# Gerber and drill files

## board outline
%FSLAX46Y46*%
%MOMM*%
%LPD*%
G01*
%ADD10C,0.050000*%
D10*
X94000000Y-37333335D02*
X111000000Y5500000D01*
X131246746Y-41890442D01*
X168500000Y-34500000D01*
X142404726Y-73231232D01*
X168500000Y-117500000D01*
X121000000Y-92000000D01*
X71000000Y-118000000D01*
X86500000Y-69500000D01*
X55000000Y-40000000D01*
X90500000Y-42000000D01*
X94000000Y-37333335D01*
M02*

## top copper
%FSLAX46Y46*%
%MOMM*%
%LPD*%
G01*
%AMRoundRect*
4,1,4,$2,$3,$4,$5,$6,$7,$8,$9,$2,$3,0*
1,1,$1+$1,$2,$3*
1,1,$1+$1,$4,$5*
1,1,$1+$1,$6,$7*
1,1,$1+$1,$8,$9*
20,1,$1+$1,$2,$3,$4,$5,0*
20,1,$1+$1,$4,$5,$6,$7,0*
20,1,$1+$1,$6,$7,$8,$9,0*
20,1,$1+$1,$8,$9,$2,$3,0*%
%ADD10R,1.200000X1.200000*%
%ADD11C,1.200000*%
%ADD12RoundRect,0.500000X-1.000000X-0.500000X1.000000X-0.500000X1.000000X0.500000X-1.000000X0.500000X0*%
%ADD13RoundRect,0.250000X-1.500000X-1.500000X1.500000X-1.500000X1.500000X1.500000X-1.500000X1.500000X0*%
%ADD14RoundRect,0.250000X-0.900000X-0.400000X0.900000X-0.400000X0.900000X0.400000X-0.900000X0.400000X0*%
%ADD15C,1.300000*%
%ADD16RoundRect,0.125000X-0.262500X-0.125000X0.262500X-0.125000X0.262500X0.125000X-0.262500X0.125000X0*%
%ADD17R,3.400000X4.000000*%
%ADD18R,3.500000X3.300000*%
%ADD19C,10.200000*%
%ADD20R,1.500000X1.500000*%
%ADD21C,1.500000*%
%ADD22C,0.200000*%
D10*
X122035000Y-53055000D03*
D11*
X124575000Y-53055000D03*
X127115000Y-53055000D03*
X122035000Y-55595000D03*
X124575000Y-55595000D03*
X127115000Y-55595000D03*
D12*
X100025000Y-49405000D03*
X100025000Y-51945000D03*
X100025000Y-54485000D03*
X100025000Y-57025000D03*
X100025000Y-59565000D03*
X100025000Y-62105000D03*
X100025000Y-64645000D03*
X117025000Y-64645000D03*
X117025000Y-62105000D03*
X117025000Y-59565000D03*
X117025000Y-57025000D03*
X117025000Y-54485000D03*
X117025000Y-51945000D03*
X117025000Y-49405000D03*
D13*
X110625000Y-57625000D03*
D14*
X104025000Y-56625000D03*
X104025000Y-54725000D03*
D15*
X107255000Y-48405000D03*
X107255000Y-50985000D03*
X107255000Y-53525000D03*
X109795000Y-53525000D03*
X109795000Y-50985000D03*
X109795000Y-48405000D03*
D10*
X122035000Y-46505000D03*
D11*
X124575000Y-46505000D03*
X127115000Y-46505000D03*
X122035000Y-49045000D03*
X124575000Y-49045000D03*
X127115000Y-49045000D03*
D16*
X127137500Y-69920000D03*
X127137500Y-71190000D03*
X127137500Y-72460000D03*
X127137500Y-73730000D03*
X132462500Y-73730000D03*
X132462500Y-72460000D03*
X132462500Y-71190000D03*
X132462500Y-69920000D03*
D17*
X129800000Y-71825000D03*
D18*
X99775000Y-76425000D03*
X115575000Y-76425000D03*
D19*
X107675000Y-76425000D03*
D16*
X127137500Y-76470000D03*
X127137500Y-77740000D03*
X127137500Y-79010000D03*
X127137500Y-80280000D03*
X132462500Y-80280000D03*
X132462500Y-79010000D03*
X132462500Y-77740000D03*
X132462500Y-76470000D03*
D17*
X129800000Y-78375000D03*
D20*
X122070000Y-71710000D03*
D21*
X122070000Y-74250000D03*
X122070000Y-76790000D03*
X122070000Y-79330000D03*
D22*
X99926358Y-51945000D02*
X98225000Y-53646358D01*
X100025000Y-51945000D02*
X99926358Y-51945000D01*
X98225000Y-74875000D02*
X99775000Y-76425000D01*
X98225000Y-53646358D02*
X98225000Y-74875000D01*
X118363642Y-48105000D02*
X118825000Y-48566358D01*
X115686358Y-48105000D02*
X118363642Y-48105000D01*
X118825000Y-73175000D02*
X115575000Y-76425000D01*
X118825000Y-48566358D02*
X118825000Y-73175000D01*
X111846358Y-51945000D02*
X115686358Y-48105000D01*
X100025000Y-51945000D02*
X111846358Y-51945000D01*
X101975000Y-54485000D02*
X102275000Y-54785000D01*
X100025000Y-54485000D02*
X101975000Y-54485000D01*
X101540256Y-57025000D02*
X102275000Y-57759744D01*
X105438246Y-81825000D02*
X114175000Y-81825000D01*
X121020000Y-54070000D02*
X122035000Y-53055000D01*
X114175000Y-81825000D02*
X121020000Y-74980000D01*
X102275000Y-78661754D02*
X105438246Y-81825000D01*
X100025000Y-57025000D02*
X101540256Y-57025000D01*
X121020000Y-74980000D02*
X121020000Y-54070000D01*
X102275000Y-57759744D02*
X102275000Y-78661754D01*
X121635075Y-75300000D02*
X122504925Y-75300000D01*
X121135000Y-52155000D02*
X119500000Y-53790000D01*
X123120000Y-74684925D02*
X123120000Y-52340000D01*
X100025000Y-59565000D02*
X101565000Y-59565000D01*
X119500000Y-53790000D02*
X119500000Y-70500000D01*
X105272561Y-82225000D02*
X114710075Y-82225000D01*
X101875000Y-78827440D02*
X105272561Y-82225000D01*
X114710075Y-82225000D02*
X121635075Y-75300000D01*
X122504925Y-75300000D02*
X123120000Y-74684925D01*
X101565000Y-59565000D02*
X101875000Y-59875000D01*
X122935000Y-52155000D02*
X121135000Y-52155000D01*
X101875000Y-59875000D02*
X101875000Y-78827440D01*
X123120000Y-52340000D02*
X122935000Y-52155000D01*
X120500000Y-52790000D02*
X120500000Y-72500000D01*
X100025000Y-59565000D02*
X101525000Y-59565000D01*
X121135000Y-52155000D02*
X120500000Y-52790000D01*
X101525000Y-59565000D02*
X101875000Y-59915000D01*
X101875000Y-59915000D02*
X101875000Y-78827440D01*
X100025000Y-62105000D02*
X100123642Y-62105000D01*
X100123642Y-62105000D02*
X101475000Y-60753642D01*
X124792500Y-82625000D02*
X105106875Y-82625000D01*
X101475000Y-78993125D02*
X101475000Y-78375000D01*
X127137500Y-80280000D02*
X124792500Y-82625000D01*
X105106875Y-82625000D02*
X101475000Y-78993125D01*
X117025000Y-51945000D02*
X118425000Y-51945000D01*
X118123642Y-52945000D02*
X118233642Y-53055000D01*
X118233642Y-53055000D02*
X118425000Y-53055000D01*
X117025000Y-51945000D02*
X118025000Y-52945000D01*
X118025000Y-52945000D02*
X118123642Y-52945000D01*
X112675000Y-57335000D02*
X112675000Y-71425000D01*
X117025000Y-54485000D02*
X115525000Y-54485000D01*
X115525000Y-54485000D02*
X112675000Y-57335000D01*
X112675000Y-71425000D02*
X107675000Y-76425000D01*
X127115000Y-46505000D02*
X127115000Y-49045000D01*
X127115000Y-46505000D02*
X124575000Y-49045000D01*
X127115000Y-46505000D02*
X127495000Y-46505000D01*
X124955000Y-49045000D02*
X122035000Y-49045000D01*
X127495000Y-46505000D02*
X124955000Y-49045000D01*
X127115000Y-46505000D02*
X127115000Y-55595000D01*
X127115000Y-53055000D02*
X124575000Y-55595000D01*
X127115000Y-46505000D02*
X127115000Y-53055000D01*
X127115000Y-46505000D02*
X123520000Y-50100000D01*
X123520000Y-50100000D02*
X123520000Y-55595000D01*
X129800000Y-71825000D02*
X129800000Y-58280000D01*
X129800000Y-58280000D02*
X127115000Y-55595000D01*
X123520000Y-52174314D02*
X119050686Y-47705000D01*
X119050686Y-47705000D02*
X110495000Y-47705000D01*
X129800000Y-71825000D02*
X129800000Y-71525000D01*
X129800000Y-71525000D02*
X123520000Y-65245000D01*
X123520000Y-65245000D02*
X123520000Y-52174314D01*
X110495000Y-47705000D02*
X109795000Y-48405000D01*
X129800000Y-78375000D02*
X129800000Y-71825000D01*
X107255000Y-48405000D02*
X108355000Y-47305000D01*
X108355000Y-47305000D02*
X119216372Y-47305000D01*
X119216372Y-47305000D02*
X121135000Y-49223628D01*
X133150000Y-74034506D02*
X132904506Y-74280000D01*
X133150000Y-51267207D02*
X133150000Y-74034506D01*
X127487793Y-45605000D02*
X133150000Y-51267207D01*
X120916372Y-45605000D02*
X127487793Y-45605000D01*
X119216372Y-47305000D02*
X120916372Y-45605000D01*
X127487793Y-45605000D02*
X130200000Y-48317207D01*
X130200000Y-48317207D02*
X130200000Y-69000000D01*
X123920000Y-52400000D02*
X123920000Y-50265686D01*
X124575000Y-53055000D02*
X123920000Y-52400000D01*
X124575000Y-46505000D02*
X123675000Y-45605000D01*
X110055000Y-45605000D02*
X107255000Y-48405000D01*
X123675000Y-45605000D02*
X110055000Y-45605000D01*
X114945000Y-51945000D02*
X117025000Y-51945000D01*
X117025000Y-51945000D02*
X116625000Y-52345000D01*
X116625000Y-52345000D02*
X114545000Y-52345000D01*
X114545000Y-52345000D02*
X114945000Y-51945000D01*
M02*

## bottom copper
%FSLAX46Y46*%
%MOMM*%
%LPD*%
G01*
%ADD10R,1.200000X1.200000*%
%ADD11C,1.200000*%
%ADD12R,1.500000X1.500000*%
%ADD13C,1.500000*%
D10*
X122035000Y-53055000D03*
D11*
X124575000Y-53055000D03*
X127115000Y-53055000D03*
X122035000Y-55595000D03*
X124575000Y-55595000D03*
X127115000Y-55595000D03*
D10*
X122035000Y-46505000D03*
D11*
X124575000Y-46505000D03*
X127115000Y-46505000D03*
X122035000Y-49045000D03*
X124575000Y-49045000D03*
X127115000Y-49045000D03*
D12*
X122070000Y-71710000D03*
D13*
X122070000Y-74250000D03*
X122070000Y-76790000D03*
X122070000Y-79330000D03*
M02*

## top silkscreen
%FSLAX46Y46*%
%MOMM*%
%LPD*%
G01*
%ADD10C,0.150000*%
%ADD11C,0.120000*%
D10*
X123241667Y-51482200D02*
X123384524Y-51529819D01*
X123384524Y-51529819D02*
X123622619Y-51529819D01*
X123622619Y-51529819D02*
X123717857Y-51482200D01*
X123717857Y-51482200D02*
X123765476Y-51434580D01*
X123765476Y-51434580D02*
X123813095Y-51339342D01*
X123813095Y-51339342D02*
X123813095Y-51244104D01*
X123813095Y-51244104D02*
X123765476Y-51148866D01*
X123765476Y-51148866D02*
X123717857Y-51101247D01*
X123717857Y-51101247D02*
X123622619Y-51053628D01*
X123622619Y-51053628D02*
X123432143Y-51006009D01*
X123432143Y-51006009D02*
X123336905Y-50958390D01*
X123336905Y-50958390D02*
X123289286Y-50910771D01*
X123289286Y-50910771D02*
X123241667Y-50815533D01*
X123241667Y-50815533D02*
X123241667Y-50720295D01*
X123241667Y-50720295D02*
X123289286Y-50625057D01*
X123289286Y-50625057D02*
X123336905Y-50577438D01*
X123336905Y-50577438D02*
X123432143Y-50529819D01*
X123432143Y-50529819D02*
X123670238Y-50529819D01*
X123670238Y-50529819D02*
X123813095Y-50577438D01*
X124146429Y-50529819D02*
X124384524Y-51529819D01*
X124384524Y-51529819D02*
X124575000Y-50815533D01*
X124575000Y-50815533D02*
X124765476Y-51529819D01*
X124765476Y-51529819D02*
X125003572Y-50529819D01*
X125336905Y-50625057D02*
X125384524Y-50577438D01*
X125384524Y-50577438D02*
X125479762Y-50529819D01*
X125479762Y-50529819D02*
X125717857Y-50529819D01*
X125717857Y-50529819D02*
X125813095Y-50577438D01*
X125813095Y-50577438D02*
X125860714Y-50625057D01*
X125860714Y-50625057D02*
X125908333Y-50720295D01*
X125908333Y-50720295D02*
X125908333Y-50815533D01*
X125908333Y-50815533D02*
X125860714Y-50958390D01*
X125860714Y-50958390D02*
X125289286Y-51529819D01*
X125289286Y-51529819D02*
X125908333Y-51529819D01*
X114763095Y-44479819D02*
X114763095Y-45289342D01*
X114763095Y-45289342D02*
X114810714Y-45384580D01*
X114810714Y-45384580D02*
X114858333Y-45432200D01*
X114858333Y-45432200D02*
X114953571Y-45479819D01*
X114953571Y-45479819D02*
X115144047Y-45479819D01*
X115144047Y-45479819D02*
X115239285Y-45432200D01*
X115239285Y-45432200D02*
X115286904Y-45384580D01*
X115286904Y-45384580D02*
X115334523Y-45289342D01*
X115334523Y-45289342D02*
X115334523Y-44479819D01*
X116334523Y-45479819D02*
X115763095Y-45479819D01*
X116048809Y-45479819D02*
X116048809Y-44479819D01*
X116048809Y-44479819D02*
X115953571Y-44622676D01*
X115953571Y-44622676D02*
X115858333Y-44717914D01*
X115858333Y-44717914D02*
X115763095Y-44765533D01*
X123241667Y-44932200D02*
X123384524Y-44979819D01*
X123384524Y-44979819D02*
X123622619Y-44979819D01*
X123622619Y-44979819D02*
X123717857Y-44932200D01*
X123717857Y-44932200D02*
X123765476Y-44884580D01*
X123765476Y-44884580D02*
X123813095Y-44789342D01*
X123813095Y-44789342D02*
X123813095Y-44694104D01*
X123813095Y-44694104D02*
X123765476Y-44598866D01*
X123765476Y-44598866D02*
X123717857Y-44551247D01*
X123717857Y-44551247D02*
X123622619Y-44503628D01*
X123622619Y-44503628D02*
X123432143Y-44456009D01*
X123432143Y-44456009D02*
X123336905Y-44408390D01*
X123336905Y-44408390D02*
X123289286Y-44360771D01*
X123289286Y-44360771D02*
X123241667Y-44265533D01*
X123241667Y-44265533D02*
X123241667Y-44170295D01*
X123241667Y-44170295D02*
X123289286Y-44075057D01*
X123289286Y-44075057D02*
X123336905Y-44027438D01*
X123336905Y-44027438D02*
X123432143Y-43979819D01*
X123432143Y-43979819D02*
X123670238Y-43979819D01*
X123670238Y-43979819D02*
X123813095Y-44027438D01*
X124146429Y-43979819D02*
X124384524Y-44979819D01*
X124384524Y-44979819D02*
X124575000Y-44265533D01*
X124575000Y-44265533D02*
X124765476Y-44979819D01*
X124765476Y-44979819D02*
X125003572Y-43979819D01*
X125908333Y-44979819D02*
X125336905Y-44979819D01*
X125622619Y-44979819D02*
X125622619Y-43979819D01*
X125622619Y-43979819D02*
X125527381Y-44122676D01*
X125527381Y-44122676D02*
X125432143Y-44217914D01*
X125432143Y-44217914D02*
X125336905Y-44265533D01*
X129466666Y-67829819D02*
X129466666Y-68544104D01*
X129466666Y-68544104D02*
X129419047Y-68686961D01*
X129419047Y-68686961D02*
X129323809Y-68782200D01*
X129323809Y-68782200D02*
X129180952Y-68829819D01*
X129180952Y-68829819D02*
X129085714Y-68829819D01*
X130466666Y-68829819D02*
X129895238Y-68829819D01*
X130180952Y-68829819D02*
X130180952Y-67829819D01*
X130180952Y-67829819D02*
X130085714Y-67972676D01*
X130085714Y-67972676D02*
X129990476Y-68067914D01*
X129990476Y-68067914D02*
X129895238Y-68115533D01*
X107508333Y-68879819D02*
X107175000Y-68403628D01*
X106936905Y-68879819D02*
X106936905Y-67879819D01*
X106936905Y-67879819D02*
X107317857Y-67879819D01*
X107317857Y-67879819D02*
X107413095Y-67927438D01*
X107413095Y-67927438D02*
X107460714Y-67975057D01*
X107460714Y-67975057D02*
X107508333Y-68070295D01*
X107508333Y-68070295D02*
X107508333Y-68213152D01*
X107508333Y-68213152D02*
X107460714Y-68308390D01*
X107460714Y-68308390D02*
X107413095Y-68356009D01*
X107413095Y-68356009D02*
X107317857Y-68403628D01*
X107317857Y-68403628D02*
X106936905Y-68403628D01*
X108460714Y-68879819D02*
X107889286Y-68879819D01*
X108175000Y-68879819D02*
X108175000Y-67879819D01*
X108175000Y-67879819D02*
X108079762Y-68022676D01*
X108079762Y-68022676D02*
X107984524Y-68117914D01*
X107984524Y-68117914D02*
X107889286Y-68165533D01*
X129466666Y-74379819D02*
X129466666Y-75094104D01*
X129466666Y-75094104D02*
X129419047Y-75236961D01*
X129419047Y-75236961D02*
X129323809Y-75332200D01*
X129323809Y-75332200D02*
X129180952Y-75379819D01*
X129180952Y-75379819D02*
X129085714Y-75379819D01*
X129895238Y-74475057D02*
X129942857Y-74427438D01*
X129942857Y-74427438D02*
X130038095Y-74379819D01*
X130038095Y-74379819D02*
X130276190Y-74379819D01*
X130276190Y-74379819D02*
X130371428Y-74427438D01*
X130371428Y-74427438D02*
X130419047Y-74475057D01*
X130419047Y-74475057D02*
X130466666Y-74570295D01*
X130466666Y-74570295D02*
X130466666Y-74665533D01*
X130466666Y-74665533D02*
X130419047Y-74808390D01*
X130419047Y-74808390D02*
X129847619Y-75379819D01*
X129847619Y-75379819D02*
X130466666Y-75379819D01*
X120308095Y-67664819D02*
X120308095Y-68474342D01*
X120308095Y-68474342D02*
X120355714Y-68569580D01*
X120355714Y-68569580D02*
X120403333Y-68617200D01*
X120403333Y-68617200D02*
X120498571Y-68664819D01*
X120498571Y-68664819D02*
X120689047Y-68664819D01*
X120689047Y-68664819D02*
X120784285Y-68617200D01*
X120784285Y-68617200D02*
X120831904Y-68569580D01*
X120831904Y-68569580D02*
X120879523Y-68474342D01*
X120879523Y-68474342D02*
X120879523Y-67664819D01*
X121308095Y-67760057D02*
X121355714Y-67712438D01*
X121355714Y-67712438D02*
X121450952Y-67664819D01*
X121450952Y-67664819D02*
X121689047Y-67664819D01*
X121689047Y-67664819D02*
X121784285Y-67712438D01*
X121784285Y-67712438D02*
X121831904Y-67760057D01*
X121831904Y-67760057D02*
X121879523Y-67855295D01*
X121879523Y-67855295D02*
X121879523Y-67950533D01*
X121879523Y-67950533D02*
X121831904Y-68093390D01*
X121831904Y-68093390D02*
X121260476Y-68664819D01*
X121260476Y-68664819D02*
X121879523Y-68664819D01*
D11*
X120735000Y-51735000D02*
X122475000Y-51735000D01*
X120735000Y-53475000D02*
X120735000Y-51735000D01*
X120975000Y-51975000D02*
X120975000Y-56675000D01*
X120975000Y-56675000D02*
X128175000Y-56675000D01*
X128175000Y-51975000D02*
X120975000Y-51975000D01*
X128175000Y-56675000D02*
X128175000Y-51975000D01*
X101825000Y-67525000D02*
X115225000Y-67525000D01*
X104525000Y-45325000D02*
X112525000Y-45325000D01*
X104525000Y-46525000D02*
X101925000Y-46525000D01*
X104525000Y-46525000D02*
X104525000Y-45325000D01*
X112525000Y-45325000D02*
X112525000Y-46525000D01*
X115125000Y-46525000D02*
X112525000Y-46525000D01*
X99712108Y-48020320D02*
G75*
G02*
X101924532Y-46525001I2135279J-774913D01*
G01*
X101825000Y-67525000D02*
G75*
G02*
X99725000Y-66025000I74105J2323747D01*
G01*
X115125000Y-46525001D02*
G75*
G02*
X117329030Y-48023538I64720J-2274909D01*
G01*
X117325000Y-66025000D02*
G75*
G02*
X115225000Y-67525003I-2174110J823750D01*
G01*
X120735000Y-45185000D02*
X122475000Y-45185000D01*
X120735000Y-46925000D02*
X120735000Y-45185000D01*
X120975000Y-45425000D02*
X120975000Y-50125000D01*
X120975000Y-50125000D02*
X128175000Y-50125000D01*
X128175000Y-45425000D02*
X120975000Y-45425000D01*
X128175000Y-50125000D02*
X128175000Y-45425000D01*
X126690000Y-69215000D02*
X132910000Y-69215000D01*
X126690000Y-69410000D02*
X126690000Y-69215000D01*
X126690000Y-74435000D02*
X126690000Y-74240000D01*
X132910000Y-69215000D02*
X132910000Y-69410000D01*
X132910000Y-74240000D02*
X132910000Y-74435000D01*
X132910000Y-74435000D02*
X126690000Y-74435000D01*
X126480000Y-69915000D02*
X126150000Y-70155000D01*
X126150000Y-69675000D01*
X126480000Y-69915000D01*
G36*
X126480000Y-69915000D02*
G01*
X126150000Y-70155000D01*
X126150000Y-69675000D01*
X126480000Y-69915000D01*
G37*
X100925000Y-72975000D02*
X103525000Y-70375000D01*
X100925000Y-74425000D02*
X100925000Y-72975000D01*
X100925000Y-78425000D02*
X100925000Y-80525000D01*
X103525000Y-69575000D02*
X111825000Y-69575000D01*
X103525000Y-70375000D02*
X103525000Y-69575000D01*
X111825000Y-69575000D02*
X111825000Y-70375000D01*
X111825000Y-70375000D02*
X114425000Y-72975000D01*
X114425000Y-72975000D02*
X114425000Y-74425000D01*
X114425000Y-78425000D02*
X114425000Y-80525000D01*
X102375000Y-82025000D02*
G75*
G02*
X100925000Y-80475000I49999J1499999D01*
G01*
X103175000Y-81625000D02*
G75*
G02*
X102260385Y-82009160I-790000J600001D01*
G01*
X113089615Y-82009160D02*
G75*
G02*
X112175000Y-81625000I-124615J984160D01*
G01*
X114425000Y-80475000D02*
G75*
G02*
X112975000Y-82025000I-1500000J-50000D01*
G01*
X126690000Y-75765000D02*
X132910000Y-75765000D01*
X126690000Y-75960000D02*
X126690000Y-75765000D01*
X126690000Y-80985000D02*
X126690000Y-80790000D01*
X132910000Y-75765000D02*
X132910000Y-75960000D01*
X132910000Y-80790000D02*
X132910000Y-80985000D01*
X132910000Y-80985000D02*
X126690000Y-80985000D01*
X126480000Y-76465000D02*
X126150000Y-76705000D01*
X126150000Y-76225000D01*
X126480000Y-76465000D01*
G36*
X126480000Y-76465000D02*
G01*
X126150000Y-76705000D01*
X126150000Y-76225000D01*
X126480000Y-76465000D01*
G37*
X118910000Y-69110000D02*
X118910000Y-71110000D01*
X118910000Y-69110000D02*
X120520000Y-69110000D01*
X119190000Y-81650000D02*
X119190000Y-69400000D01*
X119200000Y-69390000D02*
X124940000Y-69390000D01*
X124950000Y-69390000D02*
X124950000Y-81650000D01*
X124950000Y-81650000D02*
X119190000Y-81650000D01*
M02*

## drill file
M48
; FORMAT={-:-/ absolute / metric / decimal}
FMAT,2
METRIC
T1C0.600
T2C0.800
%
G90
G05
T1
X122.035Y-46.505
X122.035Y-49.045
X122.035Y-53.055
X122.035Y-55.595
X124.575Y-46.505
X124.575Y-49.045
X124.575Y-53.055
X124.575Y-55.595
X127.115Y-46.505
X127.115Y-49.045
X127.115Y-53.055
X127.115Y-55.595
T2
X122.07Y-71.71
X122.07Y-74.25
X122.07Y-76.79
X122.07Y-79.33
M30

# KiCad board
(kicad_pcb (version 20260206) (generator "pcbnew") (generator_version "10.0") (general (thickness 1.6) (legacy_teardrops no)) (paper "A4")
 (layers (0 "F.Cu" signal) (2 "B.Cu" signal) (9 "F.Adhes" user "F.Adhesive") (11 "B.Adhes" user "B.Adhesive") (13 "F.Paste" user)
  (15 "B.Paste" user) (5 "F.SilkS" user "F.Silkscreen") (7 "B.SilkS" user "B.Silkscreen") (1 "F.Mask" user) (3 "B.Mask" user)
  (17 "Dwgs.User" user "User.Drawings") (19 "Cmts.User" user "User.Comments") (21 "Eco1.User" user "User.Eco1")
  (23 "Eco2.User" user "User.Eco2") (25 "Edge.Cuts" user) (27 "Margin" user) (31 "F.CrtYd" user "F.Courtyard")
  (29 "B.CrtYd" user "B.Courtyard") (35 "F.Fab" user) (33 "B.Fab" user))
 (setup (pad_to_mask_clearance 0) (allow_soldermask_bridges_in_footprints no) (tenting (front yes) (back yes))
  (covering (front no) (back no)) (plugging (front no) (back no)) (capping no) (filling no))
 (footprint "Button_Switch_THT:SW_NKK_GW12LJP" (layer "F.Cu") (at 122.035 53.055)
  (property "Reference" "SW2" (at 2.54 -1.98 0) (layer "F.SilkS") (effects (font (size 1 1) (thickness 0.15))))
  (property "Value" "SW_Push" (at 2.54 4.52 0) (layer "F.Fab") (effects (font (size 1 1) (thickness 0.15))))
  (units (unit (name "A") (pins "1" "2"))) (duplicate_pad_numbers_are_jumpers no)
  (fp_line (start -1.3 -1.32) (end 0.44 -1.32) (stroke (width 0.12) (type solid)) (layer "F.SilkS"))
  (fp_line (start -1.3 0.42) (end -1.3 -1.32) (stroke (width 0.12) (type solid)) (layer "F.SilkS"))
  (fp_line (start -1.06 -1.08) (end -1.06 3.62) (stroke (width 0.12) (type solid)) (layer "F.SilkS"))
  (fp_line (start -1.06 3.62) (end 6.14 3.62) (stroke (width 0.12) (type solid)) (layer "F.SilkS"))
  (fp_line (start 6.14 -1.08) (end -1.06 -1.08) (stroke (width 0.12) (type solid)) (layer "F.SilkS"))
  (fp_line (start 6.14 3.62) (end 6.14 -1.08) (stroke (width 0.12) (type solid)) (layer "F.SilkS"))
  (pad "1" thru_hole rect (at 0 0) (size 1.2 1.2) (drill 0.6) (layers "*.Cu" "*.Mask") (remove_unused_layers no) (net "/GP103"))
  (pad "2" thru_hole circle (at 2.54 0) (size 1.2 1.2) (drill 0.6) (layers "*.Cu" "*.Mask") (remove_unused_layers no) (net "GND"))
  (pad "3" thru_hole circle (at 5.08 0) (size 1.2 1.2) (drill 0.6) (layers "*.Cu" "*.Mask") (remove_unused_layers no))
  (pad "4" thru_hole circle (at 0 2.54) (size 1.2 1.2) (drill 0.6) (layers "*.Cu" "*.Mask") (remove_unused_layers no))
  (pad "5" thru_hole circle (at 2.54 2.54) (size 1.2 1.2) (drill 0.6) (layers "*.Cu" "*.Mask") (remove_unused_layers no))
  (pad "6" thru_hole circle (at 5.08 2.54) (size 1.2 1.2) (drill 0.6) (layers "*.Cu" "*.Mask") (remove_unused_layers no)))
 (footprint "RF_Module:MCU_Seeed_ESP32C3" (layer "F.Cu") (at 108.525 57.025)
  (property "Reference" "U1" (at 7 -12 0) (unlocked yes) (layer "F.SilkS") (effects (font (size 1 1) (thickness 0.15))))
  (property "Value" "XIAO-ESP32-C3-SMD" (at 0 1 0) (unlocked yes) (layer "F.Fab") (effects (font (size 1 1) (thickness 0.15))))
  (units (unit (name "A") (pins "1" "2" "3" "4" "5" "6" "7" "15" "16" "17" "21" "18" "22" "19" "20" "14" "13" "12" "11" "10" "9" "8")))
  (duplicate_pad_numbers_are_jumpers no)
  (fp_line (start -6.7 10.5) (end 6.7 10.5) (stroke (width 0.12) (type default)) (layer "F.SilkS"))
  (fp_line (start -4 -11.7) (end 4 -11.7) (stroke (width 0.12) (type default)) (layer "F.SilkS"))
  (fp_line (start -4 -10.5) (end -6.6 -10.5) (stroke (width 0.12) (type default)) (layer "F.SilkS"))
  (fp_line (start -4 -10.5) (end -4 -11.7) (stroke (width 0.12) (type default)) (layer "F.SilkS"))
  (fp_line (start 4 -11.7) (end 4 -10.5) (stroke (width 0.12) (type default)) (layer "F.SilkS"))
  (fp_line (start 6.6 -10.5) (end 4 -10.5) (stroke (width 0.12) (type default)) (layer "F.SilkS"))
  (fp_arc (start -8.812892 -9.00468) (mid -7.949609 -10.111769) (end -6.600468 -10.499999) (stroke (width 0.12) (type default))
   (layer "F.SilkS"))
  (fp_arc (start -6.7 10.5) (mid -7.977232 10.068125) (end -8.8 9) (stroke (width 0.12) (type default)) (layer "F.SilkS"))
  (fp_arc (start 6.6 -10.499999) (mid 7.944325 -10.107116) (end 8.804034 -9.001464) (stroke (width 0.12) (type default)) (layer "F.SilkS"))
  (fp_arc (start 8.8 9) (mid 7.977232 10.068125) (end 6.7 10.5) (stroke (width 0.12) (type default)) (layer "F.SilkS"))
  (pad "" smd roundrect (at 1.1 -0.4) (size 1.5 1.5) (layers "F.Paste") (roundrect_rratio 0.1666666667))
  (pad "" smd roundrect (at 1.1 1.6) (size 1.5 1.5) (layers "F.Paste") (roundrect_rratio 0.1666666667))
  (pad "" smd roundrect (at 3.1 -0.4) (size 1.5 1.5) (layers "F.Paste") (roundrect_rratio 0.1666666667))
  (pad "" smd roundrect (at 3.1 1.6) (size 1.5 1.5) (layers "F.Paste") (roundrect_rratio 0.1666666667))
  (pad "1" smd roundrect (at -8.5 -7.62) (size 3 2) (layers "F.Cu" "F.Mask" "F.Paste") (roundrect_rratio 0.25)
   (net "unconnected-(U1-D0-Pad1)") (thermal_bridge_angle 45))
  (pad "2" smd roundrect (at -8.5 -5.08) (size 3 2) (layers "F.Cu" "F.Mask" "F.Paste") (roundrect_rratio 0.25) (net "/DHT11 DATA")
   (thermal_bridge_angle 45))
  (pad "3" smd roundrect (at -8.5 -2.54) (size 3 2) (layers "F.Cu" "F.Mask" "F.Paste") (roundrect_rratio 0.25) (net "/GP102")
   (thermal_bridge_angle 45))
  (pad "4" smd roundrect (at -8.5 0) (size 3 2) (layers "F.Cu" "F.Mask" "F.Paste") (roundrect_rratio 0.25) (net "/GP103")
   (thermal_bridge_angle 45))
  (pad "5" smd roundrect (at -8.5 2.54) (size 3 2) (layers "F.Cu" "F.Mask" "F.Paste") (roundrect_rratio 0.25) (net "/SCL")
   (thermal_bridge_angle 45))
  (pad "6" smd roundrect (at -8.5 5.08) (size 3 2) (layers "F.Cu" "F.Mask" "F.Paste") (roundrect_rratio 0.25) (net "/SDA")
   (thermal_bridge_angle 45))
  (pad "7" smd roundrect (at -8.5 7.62) (size 3 2) (layers "F.Cu" "F.Mask" "F.Paste") (roundrect_rratio 0.25)
   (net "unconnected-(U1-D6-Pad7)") (thermal_bridge_angle 45))
  (pad "8" smd roundrect (at 8.5 7.62) (size 3 2) (layers "F.Cu" "F.Mask" "F.Paste") (roundrect_rratio 0.25)
   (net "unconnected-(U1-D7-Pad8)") (thermal_bridge_angle 45))
  (pad "9" smd roundrect (at 8.5 5.08) (size 3 2) (layers "F.Cu" "F.Mask" "F.Paste") (roundrect_rratio 0.25)
   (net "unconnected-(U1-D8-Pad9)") (thermal_bridge_angle 45))
  (pad "10" smd roundrect (at 8.5 2.54) (size 3 2) (layers "F.Cu" "F.Mask" "F.Paste") (roundrect_rratio 0.25)
   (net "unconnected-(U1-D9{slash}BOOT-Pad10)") (thermal_bridge_angle 45))
  (pad "11" smd roundrect (at 8.5 0) (size 3 2) (layers "F.Cu" "F.Mask" "F.Paste") (roundrect_rratio 0.25)
   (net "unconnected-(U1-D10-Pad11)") (thermal_bridge_angle 45))
  (pad "12" smd roundrect (at 8.5 -2.54) (size 3 2) (layers "F.Cu" "F.Mask" "F.Paste") (roundrect_rratio 0.25) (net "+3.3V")
   (thermal_bridge_angle 45))
  (pad "13" smd roundrect (at 8.5 -5.08) (size 3 2) (layers "F.Cu" "F.Mask" "F.Paste") (roundrect_rratio 0.25) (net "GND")
   (thermal_bridge_angle 45))
  (pad "14" smd roundrect (at 8.5 -7.62) (size 3 2) (layers "F.Cu" "F.Mask" "F.Paste") (roundrect_rratio 0.25) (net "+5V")
   (thermal_bridge_angle 45))
  (pad "15" smd roundrect (at 2.1 0.6) (size 3.5 3.5) (layers "F.Cu" "F.Mask") (roundrect_rratio 0.07142857143)
   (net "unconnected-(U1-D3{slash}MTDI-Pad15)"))
  (pad "16" smd roundrect (at -4.5 -0.4) (size 2.3 1.3) (layers "F.Cu" "F.Mask" "F.Paste") (roundrect_rratio 0.1923076923)
   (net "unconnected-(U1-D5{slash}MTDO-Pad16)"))
  (pad "17" smd roundrect (at -4.5 -2.3) (size 2.3 1.3) (layers "F.Cu" "F.Mask" "F.Paste") (roundrect_rratio 0.1923076923)
   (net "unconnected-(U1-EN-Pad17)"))
  (pad "18" smd circle (at -1.27 -8.62) (size 1.3 1.3) (layers "F.Cu" "F.Mask" "F.Paste") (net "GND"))
  (pad "19" smd circle (at -1.27 -6.04) (size 1.3 1.3) (layers "F.Cu" "F.Mask" "F.Paste") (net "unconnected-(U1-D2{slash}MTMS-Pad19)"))
  (pad "20" smd circle (at -1.27 -3.5) (size 1.3 1.3) (layers "F.Cu" "F.Mask" "F.Paste") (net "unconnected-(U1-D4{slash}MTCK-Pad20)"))
  (pad "21" smd circle (at 1.27 -3.5) (size 1.3 1.3) (layers "F.Cu" "F.Mask" "F.Paste") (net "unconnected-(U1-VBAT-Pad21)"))
  (pad "22" smd circle (at 1.27 -6.04) (size 1.3 1.3) (layers "F.Cu" "F.Mask" "F.Paste") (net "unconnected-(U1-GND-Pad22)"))
  (pad "23" smd circle (at 1.27 -8.62) (size 1.3 1.3) (layers "F.Cu" "F.Mask" "F.Paste")))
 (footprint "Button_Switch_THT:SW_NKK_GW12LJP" (layer "F.Cu") (at 122.035 46.505)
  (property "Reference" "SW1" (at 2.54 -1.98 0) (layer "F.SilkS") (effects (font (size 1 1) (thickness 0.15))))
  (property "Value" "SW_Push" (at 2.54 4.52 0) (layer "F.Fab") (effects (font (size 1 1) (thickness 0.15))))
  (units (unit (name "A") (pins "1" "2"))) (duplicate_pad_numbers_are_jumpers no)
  (fp_line (start -1.3 -1.32) (end 0.44 -1.32) (stroke (width 0.12) (type solid)) (layer "F.SilkS"))
  (fp_line (start -1.3 0.42) (end -1.3 -1.32) (stroke (width 0.12) (type solid)) (layer "F.SilkS"))
  (fp_line (start -1.06 -1.08) (end -1.06 3.62) (stroke (width 0.12) (type solid)) (layer "F.SilkS"))
  (fp_line (start -1.06 3.62) (end 6.14 3.62) (stroke (width 0.12) (type solid)) (layer "F.SilkS"))
  (fp_line (start 6.14 -1.08) (end -1.06 -1.08) (stroke (width 0.12) (type solid)) (layer "F.SilkS"))
  (fp_line (start 6.14 3.62) (end 6.14 -1.08) (stroke (width 0.12) (type solid)) (layer "F.SilkS"))
  (pad "1" thru_hole rect (at 0 0) (size 1.2 1.2) (drill 0.6) (layers "*.Cu" "*.Mask") (remove_unused_layers no) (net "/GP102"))
  (pad "2" thru_hole circle (at 2.54 0) (size 1.2 1.2) (drill 0.6) (layers "*.Cu" "*.Mask") (remove_unused_layers no) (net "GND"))
  (pad "3" thru_hole circle (at 5.08 0) (size 1.2 1.2) (drill 0.6) (layers "*.Cu" "*.Mask") (remove_unused_layers no))
  (pad "4" thru_hole circle (at 0 2.54) (size 1.2 1.2) (drill 0.6) (layers "*.Cu" "*.Mask") (remove_unused_layers no))
  (pad "5" thru_hole circle (at 2.54 2.54) (size 1.2 1.2) (drill 0.6) (layers "*.Cu" "*.Mask") (remove_unused_layers no))
  (pad "6" thru_hole circle (at 5.08 2.54) (size 1.2 1.2) (drill 0.6) (layers "*.Cu" "*.Mask") (remove_unused_layers no)))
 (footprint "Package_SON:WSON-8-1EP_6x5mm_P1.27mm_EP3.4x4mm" (layer "F.Cu") (at 129.8 71.825)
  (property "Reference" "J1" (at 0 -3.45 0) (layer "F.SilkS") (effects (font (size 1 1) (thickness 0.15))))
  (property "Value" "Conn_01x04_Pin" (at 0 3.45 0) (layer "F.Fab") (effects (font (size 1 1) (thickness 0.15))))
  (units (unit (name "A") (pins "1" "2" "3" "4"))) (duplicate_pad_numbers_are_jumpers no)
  (fp_line (start -3.11 -2.61) (end 3.11 -2.61) (stroke (width 0.12) (type solid)) (layer "F.SilkS"))
  (fp_line (start -3.11 -2.415) (end -3.11 -2.61) (stroke (width 0.12) (type solid)) (layer "F.SilkS"))
  (fp_line (start -3.11 2.61) (end -3.11 2.415) (stroke (width 0.12) (type solid)) (layer "F.SilkS"))
  (fp_line (start 3.11 -2.61) (end 3.11 -2.415) (stroke (width 0.12) (type solid)) (layer "F.SilkS"))
  (fp_line (start 3.11 2.415) (end 3.11 2.61) (stroke (width 0.12) (type solid)) (layer "F.SilkS"))
  (fp_line (start 3.11 2.61) (end -3.11 2.61) (stroke (width 0.12) (type solid)) (layer "F.SilkS"))
  (fp_poly (pts (xy -3.32 -1.91) (xy -3.65 -1.67) (xy -3.65 -2.15)) (stroke (width 0.12) (type solid)) (fill yes) (layer "F.SilkS"))
  (pad "" smd roundrect (at -0.85 -1) (size 1.37 1.61) (layers "F.Paste") (roundrect_rratio 0.182482))
  (pad "" smd roundrect (at -0.85 1) (size 1.37 1.61) (layers "F.Paste") (roundrect_rratio 0.182482))
  (pad "" smd roundrect (at 0.85 -1) (size 1.37 1.61) (layers "F.Paste") (roundrect_rratio 0.182482))
  (pad "" smd roundrect (at 0.85 1) (size 1.37 1.61) (layers "F.Paste") (roundrect_rratio 0.182482))
  (pad "1" smd roundrect (at -2.6625 -1.905) (size 0.775 0.5) (layers "F.Cu" "F.Mask" "F.Paste") (roundrect_rratio 0.25) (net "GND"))
  (pad "2" smd roundrect (at -2.6625 -0.635) (size 0.775 0.5) (layers "F.Cu" "F.Mask" "F.Paste") (roundrect_rratio 0.25) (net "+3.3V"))
  (pad "3" smd roundrect (at -2.6625 0.635) (size 0.775 0.5) (layers "F.Cu" "F.Mask" "F.Paste") (roundrect_rratio 0.25) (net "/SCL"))
  (pad "4" smd roundrect (at -2.6625 1.905) (size 0.775 0.5) (layers "F.Cu" "F.Mask" "F.Paste") (roundrect_rratio 0.25) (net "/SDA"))
  (pad "5" smd roundrect (at 2.6625 1.905) (size 0.775 0.5) (layers "F.Cu" "F.Mask" "F.Paste") (roundrect_rratio 0.25))
  (pad "6" smd roundrect (at 2.6625 0.635) (size 0.775 0.5) (layers "F.Cu" "F.Mask" "F.Paste") (roundrect_rratio 0.25))
  (pad "7" smd roundrect (at 2.6625 -0.635) (size 0.775 0.5) (layers "F.Cu" "F.Mask" "F.Paste") (roundrect_rratio 0.25))
  (pad "8" smd roundrect (at 2.6625 -1.905) (size 0.775 0.5) (layers "F.Cu" "F.Mask" "F.Paste") (roundrect_rratio 0.25))
  (pad "9" smd rect (at 0 0) (size 3.4 4) (layers "F.Cu" "F.Mask") (zone_connect 2)))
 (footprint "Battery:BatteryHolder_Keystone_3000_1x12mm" (layer "F.Cu") (at 107.675 76.425)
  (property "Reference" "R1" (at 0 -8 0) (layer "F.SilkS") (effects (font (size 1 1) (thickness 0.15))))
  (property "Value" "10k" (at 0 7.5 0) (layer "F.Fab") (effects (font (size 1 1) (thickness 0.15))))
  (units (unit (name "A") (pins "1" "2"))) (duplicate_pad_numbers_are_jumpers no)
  (fp_line (start -6.75 -3.45) (end -4.15 -6.05) (stroke (width 0.12) (type solid)) (layer "F.SilkS"))
  (fp_line (start -6.75 -2) (end -6.75 -3.45) (stroke (width 0.12) (type solid)) (layer "F.SilkS"))
  (fp_line (start -6.75 2) (end -6.75 4.1) (stroke (width 0.12) (type solid)) (layer "F.SilkS"))
  (fp_line (start -4.15 -6.85) (end 4.15 -6.85) (stroke (width 0.12) (type solid)) (layer "F.SilkS"))
  (fp_line (start -4.15 -6.05) (end -4.15 -6.85) (stroke (width 0.12) (type solid)) (layer "F.SilkS"))
  (fp_line (start 4.15 -6.85) (end 4.15 -6.05) (stroke (width 0.12) (type solid)) (layer "F.SilkS"))
  (fp_line (start 4.15 -6.05) (end 6.75 -3.45) (stroke (width 0.12) (type solid)) (layer "F.SilkS"))
  (fp_line (start 6.75 -3.45) (end 6.75 -2) (stroke (width 0.12) (type solid)) (layer "F.SilkS"))
  (fp_line (start 6.75 2) (end 6.75 4.1) (stroke (width 0.12) (type solid)) (layer "F.SilkS"))
  (fp_arc (start -5.3 5.6) (mid -6.346016 5.125305) (end -6.75 4.05) (stroke (width 0.12) (type solid)) (layer "F.SilkS"))
  (fp_arc (start -4.5 5.2) (mid -4.90584 5.514615) (end -5.414615 5.58416) (stroke (width 0.12) (type solid)) (layer "F.SilkS"))
  (fp_arc (start 5.414615 5.58416) (mid 4.90584 5.514615) (end 4.5 5.2) (stroke (width 0.12) (type solid)) (layer "F.SilkS"))
  (fp_arc (start 6.75 4.05) (mid 6.346016 5.125305) (end 5.3 5.6) (stroke (width 0.12) (type solid)) (layer "F.SilkS"))
  (pad "1" smd rect (at -7.9 0) (size 3.5 3.3) (layers "F.Cu" "F.Mask" "F.Paste") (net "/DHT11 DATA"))
  (pad "1" smd rect (at 7.9 0) (size 3.5 3.3) (layers "F.Cu" "F.Mask" "F.Paste") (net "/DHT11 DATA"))
  (pad "2" smd circle (at 0 0) (size 10.2 10.2) (layers "F.Cu" "F.Mask") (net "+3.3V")))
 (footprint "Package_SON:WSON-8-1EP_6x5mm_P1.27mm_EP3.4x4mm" (layer "F.Cu") (at 129.8 78.375)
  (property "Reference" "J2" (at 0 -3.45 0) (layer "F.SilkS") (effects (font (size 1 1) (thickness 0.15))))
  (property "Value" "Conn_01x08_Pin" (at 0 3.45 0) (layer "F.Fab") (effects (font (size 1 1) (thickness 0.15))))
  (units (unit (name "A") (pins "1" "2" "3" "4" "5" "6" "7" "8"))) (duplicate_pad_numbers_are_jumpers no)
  (fp_line (start -3.11 -2.61) (end 3.11 -2.61) (stroke (width 0.12) (type solid)) (layer "F.SilkS"))
  (fp_line (start -3.11 -2.415) (end -3.11 -2.61) (stroke (width 0.12) (type solid)) (layer "F.SilkS"))
  (fp_line (start -3.11 2.61) (end -3.11 2.415) (stroke (width 0.12) (type solid)) (layer "F.SilkS"))
  (fp_line (start 3.11 -2.61) (end 3.11 -2.415) (stroke (width 0.12) (type solid)) (layer "F.SilkS"))
  (fp_line (start 3.11 2.415) (end 3.11 2.61) (stroke (width 0.12) (type solid)) (layer "F.SilkS"))
  (fp_line (start 3.11 2.61) (end -3.11 2.61) (stroke (width 0.12) (type solid)) (layer "F.SilkS"))
  (fp_poly (pts (xy -3.32 -1.91) (xy -3.65 -1.67) (xy -3.65 -2.15)) (stroke (width 0.12) (type solid)) (fill yes) (layer "F.SilkS"))
  (pad "" smd roundrect (at -0.85 -1) (size 1.37 1.61) (layers "F.Paste") (roundrect_rratio 0.182482))
  (pad "" smd roundrect (at -0.85 1) (size 1.37 1.61) (layers "F.Paste") (roundrect_rratio 0.182482))
  (pad "" smd roundrect (at 0.85 -1) (size 1.37 1.61) (layers "F.Paste") (roundrect_rratio 0.182482))
  (pad "" smd roundrect (at 0.85 1) (size 1.37 1.61) (layers "F.Paste") (roundrect_rratio 0.182482))
  (pad "1" smd roundrect (at -2.6625 -1.905) (size 0.775 0.5) (layers "F.Cu" "F.Mask" "F.Paste") (roundrect_rratio 0.25) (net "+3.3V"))
  (pad "2" smd roundrect (at -2.6625 -0.635) (size 0.775 0.5) (layers "F.Cu" "F.Mask" "F.Paste") (roundrect_rratio 0.25) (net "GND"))
  (pad "3" smd roundrect (at -2.6625 0.635) (size 0.775 0.5) (layers "F.Cu" "F.Mask" "F.Paste") (roundrect_rratio 0.25) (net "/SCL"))
  (pad "4" smd roundrect (at -2.6625 1.905) (size 0.775 0.5) (layers "F.Cu" "F.Mask" "F.Paste") (roundrect_rratio 0.25) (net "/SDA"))
  (pad "5" smd roundrect (at 2.6625 1.905) (size 0.775 0.5) (layers "F.Cu" "F.Mask" "F.Paste") (roundrect_rratio 0.25)
   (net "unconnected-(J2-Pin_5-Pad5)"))
  (pad "6" smd roundrect (at 2.6625 0.635) (size 0.775 0.5) (layers "F.Cu" "F.Mask" "F.Paste") (roundrect_rratio 0.25)
   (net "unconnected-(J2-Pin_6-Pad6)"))
  (pad "7" smd roundrect (at 2.6625 -0.635) (size 0.775 0.5) (layers "F.Cu" "F.Mask" "F.Paste") (roundrect_rratio 0.25)
   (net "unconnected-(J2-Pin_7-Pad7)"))
  (pad "8" smd roundrect (at 2.6625 -1.905) (size 0.775 0.5) (layers "F.Cu" "F.Mask" "F.Paste") (roundrect_rratio 0.25)
   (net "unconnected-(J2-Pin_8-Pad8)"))
  (pad "9" smd rect (at 0 0) (size 3.4 4) (layers "F.Cu" "F.Mask") (zone_connect 2)))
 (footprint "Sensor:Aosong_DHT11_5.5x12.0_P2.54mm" (layer "F.Cu") (at 122.07 71.71)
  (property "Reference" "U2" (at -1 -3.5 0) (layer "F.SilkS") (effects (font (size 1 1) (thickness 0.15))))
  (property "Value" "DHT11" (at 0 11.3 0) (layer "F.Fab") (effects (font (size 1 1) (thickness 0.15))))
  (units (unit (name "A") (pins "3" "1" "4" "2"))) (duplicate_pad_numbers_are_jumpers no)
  (fp_line (start -3.16 -2.6) (end -3.16 -0.6) (stroke (width 0.12) (type solid)) (layer "F.SilkS"))
  (fp_line (start -3.16 -2.6) (end -1.55 -2.6) (stroke (width 0.12) (type solid)) (layer "F.SilkS"))
  (fp_line (start -2.88 9.94) (end -2.88 -2.31) (stroke (width 0.12) (type solid)) (layer "F.SilkS"))
  (fp_line (start -2.87 -2.32) (end 2.87 -2.32) (stroke (width 0.12) (type solid)) (layer "F.SilkS"))
  (fp_line (start 2.88 -2.32) (end 2.88 9.94) (stroke (width 0.12) (type solid)) (layer "F.SilkS"))
  (fp_line (start 2.88 9.94) (end -2.88 9.94) (stroke (width 0.12) (type solid)) (layer "F.SilkS"))
  (pad "1" thru_hole rect (at 0 0) (size 1.5 1.5) (drill 0.8) (layers "*.Cu" "*.Mask") (remove_unused_layers no) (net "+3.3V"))
  (pad "2" thru_hole circle (at 0 2.54) (size 1.5 1.5) (drill 0.8) (layers "*.Cu" "*.Mask") (remove_unused_layers no) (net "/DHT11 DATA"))
  (pad "3" thru_hole circle (at 0 5.08) (size 1.5 1.5) (drill 0.8) (layers "*.Cu" "*.Mask") (remove_unused_layers no)
   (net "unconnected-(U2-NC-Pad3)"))
  (pad "4" thru_hole circle (at 0 7.62) (size 1.5 1.5) (drill 0.8) (layers "*.Cu" "*.Mask") (remove_unused_layers no) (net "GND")))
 (gr_poly
  (pts (xy 94 37.333335) (xy 111 -5.5) (xy 131.246746 41.890442) (xy 168.5 34.5) (xy 142.404726 73.231232) (xy 168.5 117.5) (xy 121 92)
   (xy 71 118) (xy 86.5 69.5) (xy 55 40) (xy 90.5 42))
  (stroke (width 0.05) (type solid)) (fill no) (layer "Edge.Cuts"))
 (segment (start 99.926358 51.945) (end 98.225 53.646358) (width 0.2) (layer "F.Cu") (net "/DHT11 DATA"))
 (segment (start 100.025 51.945) (end 99.926358 51.945) (width 0.2) (layer "F.Cu") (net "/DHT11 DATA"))
 (segment (start 98.225 74.875) (end 99.775 76.425) (width 0.2) (layer "F.Cu") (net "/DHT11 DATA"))
 (segment (start 98.225 53.646358) (end 98.225 74.875) (width 0.2) (layer "F.Cu") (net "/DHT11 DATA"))
 (segment (start 118.363642 48.105) (end 118.825 48.566358) (width 0.2) (layer "F.Cu") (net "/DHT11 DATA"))
 (segment (start 115.686358 48.105) (end 118.363642 48.105) (width 0.2) (layer "F.Cu") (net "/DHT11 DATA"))
 (segment (start 118.825 73.175) (end 115.575 76.425) (width 0.2) (layer "F.Cu") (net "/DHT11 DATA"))
 (segment (start 118.825 48.566358) (end 118.825 73.175) (width 0.2) (layer "F.Cu") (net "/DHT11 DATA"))
 (segment (start 111.846358 51.945) (end 115.686358 48.105) (width 0.2) (layer "F.Cu") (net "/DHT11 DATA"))
 (segment (start 100.025 51.945) (end 111.846358 51.945) (width 0.2) (layer "F.Cu") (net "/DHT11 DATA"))
 (segment (start 101.975 54.485) (end 102.275 54.785) (width 0.2) (layer "F.Cu") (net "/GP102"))
 (segment (start 100.025 54.485) (end 101.975 54.485) (width 0.2) (layer "F.Cu") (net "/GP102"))
 (segment (start 101.540256 57.025) (end 102.275 57.759744) (width 0.2) (layer "F.Cu") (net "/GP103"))
 (segment (start 105.438246 81.825) (end 114.175 81.825) (width 0.2) (layer "F.Cu") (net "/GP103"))
 (segment (start 121.02 54.07) (end 122.035 53.055) (width 0.2) (layer "F.Cu") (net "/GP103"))
 (segment (start 114.175 81.825) (end 121.02 74.98) (width 0.2) (layer "F.Cu") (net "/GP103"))
 (segment (start 102.275 78.661754) (end 105.438246 81.825) (width 0.2) (layer "F.Cu") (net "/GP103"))
 (segment (start 100.025 57.025) (end 101.540256 57.025) (width 0.2) (layer "F.Cu") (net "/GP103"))
 (segment (start 121.02 74.98) (end 121.02 54.07) (width 0.2) (layer "F.Cu") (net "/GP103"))
 (segment (start 102.275 57.759744) (end 102.275 78.661754) (width 0.2) (layer "F.Cu") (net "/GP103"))
 (segment (start 121.635075 75.3) (end 122.504925 75.3) (width 0.2) (layer "F.Cu") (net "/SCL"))
 (segment (start 121.135 52.155) (end 119.5 53.79) (width 0.2) (layer "F.Cu") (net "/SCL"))
 (segment (start 123.12 74.684925) (end 123.12 52.34) (width 0.2) (layer "F.Cu") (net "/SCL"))
 (segment (start 100.025 59.565) (end 101.565 59.565) (width 0.2) (layer "F.Cu") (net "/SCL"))
 (segment (start 119.5 53.79) (end 119.5 70.5) (width 0.2) (layer "F.Cu") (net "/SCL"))
 (segment (start 105.272561 82.225) (end 114.710075 82.225) (width 0.2) (layer "F.Cu") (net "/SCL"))
 (segment (start 101.875 78.82744) (end 105.272561 82.225) (width 0.2) (layer "F.Cu") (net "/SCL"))
 (segment (start 114.710075 82.225) (end 121.635075 75.3) (width 0.2) (layer "F.Cu") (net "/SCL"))
 (segment (start 122.504925 75.3) (end 123.12 74.684925) (width 0.2) (layer "F.Cu") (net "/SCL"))
 (segment (start 101.565 59.565) (end 101.875 59.875) (width 0.2) (layer "F.Cu") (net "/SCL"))
 (segment (start 122.935 52.155) (end 121.135 52.155) (width 0.2) (layer "F.Cu") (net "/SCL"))
 (segment (start 101.875 59.875) (end 101.875 78.82744) (width 0.2) (layer "F.Cu") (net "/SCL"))
 (segment (start 123.12 52.34) (end 122.935 52.155) (width 0.2) (layer "F.Cu") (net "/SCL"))
 (segment (start 120.5 52.79) (end 120.5 72.5) (width 0.2) (layer "F.Cu") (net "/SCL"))
 (segment (start 100.025 59.565) (end 101.525 59.565) (width 0.2) (layer "F.Cu") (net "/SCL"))
 (segment (start 121.135 52.155) (end 120.5 52.79) (width 0.2) (layer "F.Cu") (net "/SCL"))
 (segment (start 101.525 59.565) (end 101.875 59.915) (width 0.2) (layer "F.Cu") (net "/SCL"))
 (segment (start 101.875 59.915) (end 101.875 78.82744) (width 0.2) (layer "F.Cu") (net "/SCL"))
 (segment (start 100.025 62.105) (end 100.123642 62.105) (width 0.2) (layer "F.Cu") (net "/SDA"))
 (segment (start 100.123642 62.105) (end 101.475 60.753642) (width 0.2) (layer "F.Cu") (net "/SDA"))
 (segment (start 124.7925 82.625) (end 105.106875 82.625) (width 0.2) (layer "F.Cu") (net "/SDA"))
 (segment (start 101.475 78.993125) (end 101.475 78.375) (width 0.2) (layer "F.Cu") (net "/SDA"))
 (segment (start 127.1375 80.28) (end 124.7925 82.625) (width 0.2) (layer "F.Cu") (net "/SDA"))
 (segment (start 105.106875 82.625) (end 101.475 78.993125) (width 0.2) (layer "F.Cu") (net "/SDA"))
 (segment (start 117.025 51.945) (end 118.425 51.945) (width 0.2) (layer "F.Cu") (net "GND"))
 (segment (start 118.123642 52.945) (end 118.233642 53.055) (width 0.2) (layer "F.Cu") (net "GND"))
 (segment (start 118.233642 53.055) (end 118.425 53.055) (width 0.2) (layer "F.Cu") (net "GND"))
 (segment (start 117.025 51.945) (end 118.025 52.945) (width 0.2) (layer "F.Cu") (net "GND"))
 (segment (start 118.025 52.945) (end 118.123642 52.945) (width 0.2) (layer "F.Cu") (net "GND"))
 (segment (start 112.675 57.335) (end 112.675 71.425) (width 0.2) (layer "F.Cu") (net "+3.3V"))
 (segment (start 117.025 54.485) (end 115.525 54.485) (width 0.2) (layer "F.Cu") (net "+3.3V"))
 (segment (start 115.525 54.485) (end 112.675 57.335) (width 0.2) (layer "F.Cu") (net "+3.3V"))
 (segment (start 112.675 71.425) (end 107.675 76.425) (width 0.2) (layer "F.Cu") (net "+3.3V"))
 (segment (start 127.115 46.505) (end 127.115 49.045) (width 0.2) (layer "F.Cu") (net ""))
 (segment (start 127.115 46.505) (end 124.575 49.045) (width 0.2) (layer "F.Cu") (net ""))
 (segment (start 127.115 46.505) (end 127.495 46.505) (width 0.2) (layer "F.Cu") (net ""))
 (segment (start 124.955 49.045) (end 122.035 49.045) (width 0.2) (layer "F.Cu") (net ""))
 (segment (start 127.495 46.505) (end 124.955 49.045) (width 0.2) (layer "F.Cu") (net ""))
 (segment (start 127.115 46.505) (end 127.115 55.595) (width 0.2) (layer "F.Cu") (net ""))
 (segment (start 127.115 53.055) (end 124.575 55.595) (width 0.2) (layer "F.Cu") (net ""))
 (segment (start 127.115 46.505) (end 127.115 53.055) (width 0.2) (layer "F.Cu") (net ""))
 (segment (start 127.115 46.505) (end 123.52 50.1) (width 0.2) (layer "F.Cu") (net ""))
 (segment (start 123.52 50.1) (end 123.52 55.595) (width 0.2) (layer "F.Cu") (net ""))
 (segment (start 129.8 71.825) (end 129.8 58.28) (width 0.2) (layer "F.Cu") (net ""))
 (segment (start 129.8 58.28) (end 127.115 55.595) (width 0.2) (layer "F.Cu") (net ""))
 (segment (start 123.52 52.174314) (end 119.050686 47.705) (width 0.2) (layer "F.Cu") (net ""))
 (segment (start 119.050686 47.705) (end 110.495 47.705) (width 0.2) (layer "F.Cu") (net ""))
 (segment (start 129.8 71.825) (end 129.8 71.525) (width 0.2) (layer "F.Cu") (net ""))
 (segment (start 129.8 71.525) (end 123.52 65.245) (width 0.2) (layer "F.Cu") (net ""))
 (segment (start 123.52 65.245) (end 123.52 52.174314) (width 0.2) (layer "F.Cu") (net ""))
 (segment (start 110.495 47.705) (end 109.795 48.405) (width 0.2) (layer "F.Cu") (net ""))
 (segment (start 129.8 78.375) (end 129.8 71.825) (width 0.2) (layer "F.Cu") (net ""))
 (segment (start 107.255 48.405) (end 108.355 47.305) (width 0.2) (layer "F.Cu") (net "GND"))
 (segment (start 108.355 47.305) (end 119.216372 47.305) (width 0.2) (layer "F.Cu") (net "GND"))
 (segment (start 119.216372 47.305) (end 121.135 49.223628) (width 0.2) (layer "F.Cu") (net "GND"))
 (segment (start 133.15 74.034506) (end 132.904506 74.28) (width 0.2) (layer "F.Cu") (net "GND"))
 (segment (start 133.15 51.267207) (end 133.15 74.034506) (width 0.2) (layer "F.Cu") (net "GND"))
 (segment (start 127.487793 45.605) (end 133.15 51.267207) (width 0.2) (layer "F.Cu") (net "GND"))
 (segment (start 120.916372 45.605) (end 127.487793 45.605) (width 0.2) (layer "F.Cu") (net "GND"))
 (segment (start 119.216372 47.305) (end 120.916372 45.605) (width 0.2) (layer "F.Cu") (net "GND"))
 (segment (start 127.487793 45.605) (end 130.2 48.317207) (width 0.2) (layer "F.Cu") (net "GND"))
 (segment (start 130.2 48.317207) (end 130.2 69) (width 0.2) (layer "F.Cu") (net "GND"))
 (segment (start 123.92 52.4) (end 123.92 50.265686) (width 0.2) (layer "F.Cu") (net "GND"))
 (segment (start 124.575 53.055) (end 123.92 52.4) (width 0.2) (layer "F.Cu") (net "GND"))
 (segment (start 124.575 46.505) (end 123.675 45.605) (width 0.2) (layer "F.Cu") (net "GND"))
 (segment (start 110.055 45.605) (end 107.255 48.405) (width 0.2) (layer "F.Cu") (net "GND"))
 (segment (start 123.675 45.605) (end 110.055 45.605) (width 0.2) (layer "F.Cu") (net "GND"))
 (segment (start 114.945 51.945) (end 117.025 51.945) (width 0.2) (layer "F.Cu") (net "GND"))
 (segment (start 117.025 51.945) (end 116.625 52.345) (width 0.2) (layer "F.Cu") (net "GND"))
 (segment (start 116.625 52.345) (end 114.545 52.345) (width 0.2) (layer "F.Cu") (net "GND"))
 (segment (start 114.545 52.345) (end 114.945 51.945) (width 0.2) (layer "F.Cu") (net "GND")))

